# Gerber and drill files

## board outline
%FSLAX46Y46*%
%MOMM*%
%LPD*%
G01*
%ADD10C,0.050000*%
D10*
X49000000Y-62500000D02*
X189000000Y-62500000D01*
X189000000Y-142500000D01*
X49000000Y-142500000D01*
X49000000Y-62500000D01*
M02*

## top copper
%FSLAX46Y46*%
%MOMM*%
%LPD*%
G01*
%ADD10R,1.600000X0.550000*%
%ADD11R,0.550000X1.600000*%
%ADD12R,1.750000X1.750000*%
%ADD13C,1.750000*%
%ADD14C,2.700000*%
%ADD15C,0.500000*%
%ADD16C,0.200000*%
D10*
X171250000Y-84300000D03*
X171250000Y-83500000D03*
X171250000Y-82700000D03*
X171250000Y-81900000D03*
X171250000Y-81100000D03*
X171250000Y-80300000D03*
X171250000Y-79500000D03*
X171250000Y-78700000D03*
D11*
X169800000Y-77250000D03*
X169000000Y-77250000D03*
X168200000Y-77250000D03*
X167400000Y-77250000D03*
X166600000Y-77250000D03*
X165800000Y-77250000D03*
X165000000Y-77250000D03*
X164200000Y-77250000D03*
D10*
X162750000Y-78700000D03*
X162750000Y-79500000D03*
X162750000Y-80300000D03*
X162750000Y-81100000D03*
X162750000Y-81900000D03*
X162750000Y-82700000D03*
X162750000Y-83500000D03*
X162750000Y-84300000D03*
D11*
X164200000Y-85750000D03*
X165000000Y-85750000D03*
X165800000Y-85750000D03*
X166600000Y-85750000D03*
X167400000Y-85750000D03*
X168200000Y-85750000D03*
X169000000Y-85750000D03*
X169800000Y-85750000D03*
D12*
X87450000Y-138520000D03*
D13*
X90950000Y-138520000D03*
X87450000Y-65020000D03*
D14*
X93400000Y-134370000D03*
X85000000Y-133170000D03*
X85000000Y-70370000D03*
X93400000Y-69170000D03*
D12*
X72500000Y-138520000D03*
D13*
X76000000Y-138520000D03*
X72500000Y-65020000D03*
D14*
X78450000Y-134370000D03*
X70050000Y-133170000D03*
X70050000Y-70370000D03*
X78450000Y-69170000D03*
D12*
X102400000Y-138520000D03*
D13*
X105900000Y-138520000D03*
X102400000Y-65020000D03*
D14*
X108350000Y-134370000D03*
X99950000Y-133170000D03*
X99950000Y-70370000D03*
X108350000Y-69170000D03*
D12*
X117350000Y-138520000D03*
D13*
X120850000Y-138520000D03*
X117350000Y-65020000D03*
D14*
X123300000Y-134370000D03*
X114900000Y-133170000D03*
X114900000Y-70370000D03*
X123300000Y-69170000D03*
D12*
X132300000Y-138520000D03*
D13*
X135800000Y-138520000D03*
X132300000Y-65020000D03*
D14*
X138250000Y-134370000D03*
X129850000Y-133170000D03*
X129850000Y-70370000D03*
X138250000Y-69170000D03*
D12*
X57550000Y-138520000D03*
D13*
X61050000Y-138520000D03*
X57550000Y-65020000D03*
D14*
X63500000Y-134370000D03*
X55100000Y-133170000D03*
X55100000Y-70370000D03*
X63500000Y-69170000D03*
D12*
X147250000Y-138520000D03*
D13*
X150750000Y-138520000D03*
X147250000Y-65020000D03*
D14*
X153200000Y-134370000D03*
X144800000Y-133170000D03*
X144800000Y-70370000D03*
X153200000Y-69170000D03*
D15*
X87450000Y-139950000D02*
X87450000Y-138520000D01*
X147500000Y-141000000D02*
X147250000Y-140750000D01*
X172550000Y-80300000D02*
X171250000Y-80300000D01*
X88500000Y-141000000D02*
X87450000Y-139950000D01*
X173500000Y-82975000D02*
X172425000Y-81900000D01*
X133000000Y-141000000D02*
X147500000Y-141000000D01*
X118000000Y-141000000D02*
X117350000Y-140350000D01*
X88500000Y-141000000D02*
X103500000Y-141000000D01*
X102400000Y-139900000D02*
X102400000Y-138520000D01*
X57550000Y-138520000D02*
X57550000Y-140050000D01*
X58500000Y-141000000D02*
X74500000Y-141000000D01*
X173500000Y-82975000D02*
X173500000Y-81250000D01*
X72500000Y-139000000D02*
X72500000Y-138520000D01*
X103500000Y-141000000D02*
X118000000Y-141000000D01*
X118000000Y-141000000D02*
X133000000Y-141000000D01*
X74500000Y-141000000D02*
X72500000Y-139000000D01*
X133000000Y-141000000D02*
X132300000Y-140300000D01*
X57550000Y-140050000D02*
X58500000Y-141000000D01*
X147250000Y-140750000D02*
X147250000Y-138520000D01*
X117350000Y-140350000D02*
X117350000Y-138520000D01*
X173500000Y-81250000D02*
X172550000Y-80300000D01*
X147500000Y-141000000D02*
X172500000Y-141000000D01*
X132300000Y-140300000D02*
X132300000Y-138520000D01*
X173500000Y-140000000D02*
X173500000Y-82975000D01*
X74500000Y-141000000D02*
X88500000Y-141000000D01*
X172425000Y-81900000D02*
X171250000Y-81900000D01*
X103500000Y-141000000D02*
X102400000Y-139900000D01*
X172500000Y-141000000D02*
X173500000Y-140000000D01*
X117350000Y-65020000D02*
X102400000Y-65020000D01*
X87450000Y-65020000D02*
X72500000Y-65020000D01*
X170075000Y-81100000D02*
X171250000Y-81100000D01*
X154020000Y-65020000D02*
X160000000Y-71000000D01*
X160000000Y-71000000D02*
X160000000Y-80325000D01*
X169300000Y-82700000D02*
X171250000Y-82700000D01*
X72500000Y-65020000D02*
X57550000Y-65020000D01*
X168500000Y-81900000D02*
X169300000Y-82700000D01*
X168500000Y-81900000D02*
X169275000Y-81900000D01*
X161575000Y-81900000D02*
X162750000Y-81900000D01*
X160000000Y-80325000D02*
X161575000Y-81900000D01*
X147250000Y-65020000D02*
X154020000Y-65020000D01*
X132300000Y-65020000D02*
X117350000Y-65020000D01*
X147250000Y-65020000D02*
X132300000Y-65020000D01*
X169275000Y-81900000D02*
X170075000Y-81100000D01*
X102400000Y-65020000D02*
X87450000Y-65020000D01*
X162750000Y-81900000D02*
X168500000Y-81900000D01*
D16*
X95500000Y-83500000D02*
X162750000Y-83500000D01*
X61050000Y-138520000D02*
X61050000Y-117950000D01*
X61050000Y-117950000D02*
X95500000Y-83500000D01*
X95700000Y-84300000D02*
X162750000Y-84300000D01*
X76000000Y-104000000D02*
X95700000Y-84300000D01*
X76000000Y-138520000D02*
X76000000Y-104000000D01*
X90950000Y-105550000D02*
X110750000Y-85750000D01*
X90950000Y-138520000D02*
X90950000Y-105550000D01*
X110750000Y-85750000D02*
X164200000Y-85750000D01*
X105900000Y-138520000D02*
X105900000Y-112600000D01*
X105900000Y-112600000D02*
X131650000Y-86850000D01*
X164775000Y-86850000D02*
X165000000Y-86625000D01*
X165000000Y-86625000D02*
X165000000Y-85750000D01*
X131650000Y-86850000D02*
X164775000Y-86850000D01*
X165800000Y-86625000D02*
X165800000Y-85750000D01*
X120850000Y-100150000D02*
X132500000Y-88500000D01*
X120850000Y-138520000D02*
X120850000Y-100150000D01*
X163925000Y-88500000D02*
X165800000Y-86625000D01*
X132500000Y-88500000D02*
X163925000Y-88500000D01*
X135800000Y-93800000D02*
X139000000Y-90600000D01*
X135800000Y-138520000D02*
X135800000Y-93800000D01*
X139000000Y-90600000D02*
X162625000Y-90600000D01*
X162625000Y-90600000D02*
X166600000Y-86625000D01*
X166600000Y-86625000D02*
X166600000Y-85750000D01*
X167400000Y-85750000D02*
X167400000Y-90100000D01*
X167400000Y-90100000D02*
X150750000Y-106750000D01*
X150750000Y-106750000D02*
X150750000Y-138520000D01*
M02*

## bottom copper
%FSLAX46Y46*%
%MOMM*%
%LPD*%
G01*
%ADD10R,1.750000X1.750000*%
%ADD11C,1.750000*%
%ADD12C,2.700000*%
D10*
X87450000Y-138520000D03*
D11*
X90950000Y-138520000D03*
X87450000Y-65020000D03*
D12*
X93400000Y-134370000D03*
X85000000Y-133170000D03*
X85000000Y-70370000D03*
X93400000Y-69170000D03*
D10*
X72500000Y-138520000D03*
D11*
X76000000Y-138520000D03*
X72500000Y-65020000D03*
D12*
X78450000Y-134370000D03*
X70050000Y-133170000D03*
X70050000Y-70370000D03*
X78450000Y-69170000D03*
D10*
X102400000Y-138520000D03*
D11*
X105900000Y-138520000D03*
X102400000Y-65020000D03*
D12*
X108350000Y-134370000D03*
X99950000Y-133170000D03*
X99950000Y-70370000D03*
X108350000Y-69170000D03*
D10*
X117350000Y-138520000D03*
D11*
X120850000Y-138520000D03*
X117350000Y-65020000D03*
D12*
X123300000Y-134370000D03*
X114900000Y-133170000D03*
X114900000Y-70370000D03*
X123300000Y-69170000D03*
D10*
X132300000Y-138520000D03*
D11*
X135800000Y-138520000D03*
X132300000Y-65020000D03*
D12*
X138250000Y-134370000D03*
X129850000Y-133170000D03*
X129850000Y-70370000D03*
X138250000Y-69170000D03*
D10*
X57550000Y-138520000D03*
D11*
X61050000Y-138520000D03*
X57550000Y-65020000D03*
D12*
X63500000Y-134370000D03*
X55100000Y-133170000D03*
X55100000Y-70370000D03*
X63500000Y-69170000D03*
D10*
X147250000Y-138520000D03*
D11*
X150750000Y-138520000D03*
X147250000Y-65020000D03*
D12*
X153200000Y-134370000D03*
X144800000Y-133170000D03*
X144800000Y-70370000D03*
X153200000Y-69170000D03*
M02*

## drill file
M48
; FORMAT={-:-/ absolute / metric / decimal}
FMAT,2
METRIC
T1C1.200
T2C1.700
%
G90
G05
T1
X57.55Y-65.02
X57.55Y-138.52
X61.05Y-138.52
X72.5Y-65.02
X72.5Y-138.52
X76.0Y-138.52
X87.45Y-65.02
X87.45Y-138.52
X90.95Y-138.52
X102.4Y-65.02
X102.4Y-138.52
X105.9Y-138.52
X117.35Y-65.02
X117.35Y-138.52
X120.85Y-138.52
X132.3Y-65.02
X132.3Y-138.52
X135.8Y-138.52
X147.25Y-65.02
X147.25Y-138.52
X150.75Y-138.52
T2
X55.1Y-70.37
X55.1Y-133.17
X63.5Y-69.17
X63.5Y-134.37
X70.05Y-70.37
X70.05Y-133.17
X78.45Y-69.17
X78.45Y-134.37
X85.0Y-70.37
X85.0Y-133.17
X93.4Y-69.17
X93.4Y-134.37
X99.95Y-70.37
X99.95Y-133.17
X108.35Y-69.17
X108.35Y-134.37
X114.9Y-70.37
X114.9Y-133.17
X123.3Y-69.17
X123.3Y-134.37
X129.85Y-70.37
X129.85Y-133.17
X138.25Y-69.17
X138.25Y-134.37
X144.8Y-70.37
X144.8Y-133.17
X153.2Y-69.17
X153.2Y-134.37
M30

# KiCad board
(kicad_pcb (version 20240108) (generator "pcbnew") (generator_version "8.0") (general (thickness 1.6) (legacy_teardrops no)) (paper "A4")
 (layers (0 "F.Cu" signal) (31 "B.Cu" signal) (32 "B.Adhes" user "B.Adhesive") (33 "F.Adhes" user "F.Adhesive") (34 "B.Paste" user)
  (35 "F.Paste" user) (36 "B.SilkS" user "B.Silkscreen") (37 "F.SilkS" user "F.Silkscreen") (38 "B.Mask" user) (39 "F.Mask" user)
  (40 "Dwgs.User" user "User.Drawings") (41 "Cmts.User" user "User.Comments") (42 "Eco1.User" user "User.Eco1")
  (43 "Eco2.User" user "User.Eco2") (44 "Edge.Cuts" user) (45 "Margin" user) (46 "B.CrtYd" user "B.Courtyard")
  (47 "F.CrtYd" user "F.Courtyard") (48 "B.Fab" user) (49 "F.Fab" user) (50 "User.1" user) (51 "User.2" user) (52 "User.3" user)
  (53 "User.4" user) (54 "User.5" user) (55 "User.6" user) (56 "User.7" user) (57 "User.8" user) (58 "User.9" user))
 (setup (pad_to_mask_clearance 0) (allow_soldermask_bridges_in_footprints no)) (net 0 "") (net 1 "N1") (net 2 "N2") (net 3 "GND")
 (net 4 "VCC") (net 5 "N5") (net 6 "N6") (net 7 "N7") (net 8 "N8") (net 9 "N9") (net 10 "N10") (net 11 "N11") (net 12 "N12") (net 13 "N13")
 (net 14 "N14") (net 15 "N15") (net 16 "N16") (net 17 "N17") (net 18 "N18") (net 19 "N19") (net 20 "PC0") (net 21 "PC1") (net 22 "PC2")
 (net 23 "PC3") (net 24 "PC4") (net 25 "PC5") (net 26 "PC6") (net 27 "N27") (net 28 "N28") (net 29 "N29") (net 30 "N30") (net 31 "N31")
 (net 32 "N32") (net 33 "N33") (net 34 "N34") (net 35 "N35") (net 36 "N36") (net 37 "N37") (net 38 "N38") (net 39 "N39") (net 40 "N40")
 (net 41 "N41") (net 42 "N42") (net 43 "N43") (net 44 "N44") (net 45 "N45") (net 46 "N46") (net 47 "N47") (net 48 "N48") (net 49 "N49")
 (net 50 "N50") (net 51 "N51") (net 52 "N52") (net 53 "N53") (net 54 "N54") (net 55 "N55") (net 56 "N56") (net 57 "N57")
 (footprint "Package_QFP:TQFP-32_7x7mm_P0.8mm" (layer "F.Cu") (at 167 81.5 180)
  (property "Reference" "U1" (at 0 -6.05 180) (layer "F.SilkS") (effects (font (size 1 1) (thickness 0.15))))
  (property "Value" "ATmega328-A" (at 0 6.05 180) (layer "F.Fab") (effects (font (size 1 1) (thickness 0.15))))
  (pad "1" smd rect (at -4.25 -2.8 180) (size 1.6 0.55) (layers "F.Cu" "F.Paste" "F.Mask") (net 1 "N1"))
  (pad "2" smd rect (at -4.25 -2 180) (size 1.6 0.55) (layers "F.Cu" "F.Paste" "F.Mask") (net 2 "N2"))
  (pad "3" smd rect (at -4.25 -1.2 180) (size 1.6 0.55) (layers "F.Cu" "F.Paste" "F.Mask") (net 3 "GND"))
  (pad "4" smd rect (at -4.25 -0.4 180) (size 1.6 0.55) (layers "F.Cu" "F.Paste" "F.Mask") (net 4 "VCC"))
  (pad "5" smd rect (at -4.25 0.4 180) (size 1.6 0.55) (layers "F.Cu" "F.Paste" "F.Mask") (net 3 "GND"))
  (pad "6" smd rect (at -4.25 1.2 180) (size 1.6 0.55) (layers "F.Cu" "F.Paste" "F.Mask") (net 4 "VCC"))
  (pad "7" smd rect (at -4.25 2 180) (size 1.6 0.55) (layers "F.Cu" "F.Paste" "F.Mask") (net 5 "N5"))
  (pad "8" smd rect (at -4.25 2.8 180) (size 1.6 0.55) (layers "F.Cu" "F.Paste" "F.Mask") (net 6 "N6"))
  (pad "9" smd rect (at -2.8 4.25 270) (size 1.6 0.55) (layers "F.Cu" "F.Paste" "F.Mask") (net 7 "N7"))
  (pad "10" smd rect (at -2 4.25 270) (size 1.6 0.55) (layers "F.Cu" "F.Paste" "F.Mask") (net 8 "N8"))
  (pad "11" smd rect (at -1.2 4.25 270) (size 1.6 0.55) (layers "F.Cu" "F.Paste" "F.Mask") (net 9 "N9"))
  (pad "12" smd rect (at -0.4 4.25 270) (size 1.6 0.55) (layers "F.Cu" "F.Paste" "F.Mask") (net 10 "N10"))
  (pad "13" smd rect (at 0.4 4.25 270) (size 1.6 0.55) (layers "F.Cu" "F.Paste" "F.Mask") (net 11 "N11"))
  (pad "14" smd rect (at 1.2 4.25 270) (size 1.6 0.55) (layers "F.Cu" "F.Paste" "F.Mask") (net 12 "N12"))
  (pad "15" smd rect (at 2 4.25 270) (size 1.6 0.55) (layers "F.Cu" "F.Paste" "F.Mask") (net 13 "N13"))
  (pad "16" smd rect (at 2.8 4.25 270) (size 1.6 0.55) (layers "F.Cu" "F.Paste" "F.Mask") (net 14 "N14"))
  (pad "17" smd rect (at 4.25 2.8 180) (size 1.6 0.55) (layers "F.Cu" "F.Paste" "F.Mask") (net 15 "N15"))
  (pad "18" smd rect (at 4.25 2 180) (size 1.6 0.55) (layers "F.Cu" "F.Paste" "F.Mask") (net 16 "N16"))
  (pad "19" smd rect (at 4.25 1.2 180) (size 1.6 0.55) (layers "F.Cu" "F.Paste" "F.Mask") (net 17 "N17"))
  (pad "20" smd rect (at 4.25 0.4 180) (size 1.6 0.55) (layers "F.Cu" "F.Paste" "F.Mask") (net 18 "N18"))
  (pad "21" smd rect (at 4.25 -0.4 180) (size 1.6 0.55) (layers "F.Cu" "F.Paste" "F.Mask") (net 3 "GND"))
  (pad "22" smd rect (at 4.25 -1.2 180) (size 1.6 0.55) (layers "F.Cu" "F.Paste" "F.Mask") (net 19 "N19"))
  (pad "23" smd rect (at 4.25 -2 180) (size 1.6 0.55) (layers "F.Cu" "F.Paste" "F.Mask") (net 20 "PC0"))
  (pad "24" smd rect (at 4.25 -2.8 180) (size 1.6 0.55) (layers "F.Cu" "F.Paste" "F.Mask") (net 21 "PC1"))
  (pad "25" smd rect (at 2.8 -4.25 270) (size 1.6 0.55) (layers "F.Cu" "F.Paste" "F.Mask") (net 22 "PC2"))
  (pad "26" smd rect (at 2 -4.25 270) (size 1.6 0.55) (layers "F.Cu" "F.Paste" "F.Mask") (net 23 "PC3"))
  (pad "27" smd rect (at 1.2 -4.25 270) (size 1.6 0.55) (layers "F.Cu" "F.Paste" "F.Mask") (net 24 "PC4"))
  (pad "28" smd rect (at 0.4 -4.25 270) (size 1.6 0.55) (layers "F.Cu" "F.Paste" "F.Mask") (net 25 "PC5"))
  (pad "29" smd rect (at -0.4 -4.25 270) (size 1.6 0.55) (layers "F.Cu" "F.Paste" "F.Mask") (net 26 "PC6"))
  (pad "30" smd rect (at -1.2 -4.25 270) (size 1.6 0.55) (layers "F.Cu" "F.Paste" "F.Mask") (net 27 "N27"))
  (pad "31" smd rect (at -2 -4.25 270) (size 1.6 0.55) (layers "F.Cu" "F.Paste" "F.Mask") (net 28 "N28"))
  (pad "32" smd rect (at -2.8 -4.25 270) (size 1.6 0.55) (layers "F.Cu" "F.Paste" "F.Mask") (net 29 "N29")))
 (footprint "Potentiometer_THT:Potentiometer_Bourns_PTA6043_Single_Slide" (layer "F.Cu") (at 87.45 138.52 90)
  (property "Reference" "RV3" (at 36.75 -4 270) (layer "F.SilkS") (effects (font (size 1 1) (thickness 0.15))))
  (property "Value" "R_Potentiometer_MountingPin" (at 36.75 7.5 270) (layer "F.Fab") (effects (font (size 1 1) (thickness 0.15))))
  (pad "1" thru_hole rect (at 0 0 90) (size 1.75 1.75) (drill 1.2) (layers "*.Cu" "*.Mask") (remove_unused_layers no) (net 4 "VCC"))
  (pad "2" thru_hole circle (at 0 3.5 90) (size 1.75 1.75) (drill 1.2) (layers "*.Cu" "*.Mask") (remove_unused_layers no) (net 22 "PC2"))
  (pad "3" thru_hole circle (at 73.5 0 90) (size 1.75 1.75) (drill 1.2) (layers "*.Cu" "*.Mask") (remove_unused_layers no) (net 3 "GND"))
  (pad "MP" thru_hole circle (at 4.15 5.95 90) (size 2.7 2.7) (drill 1.7) (layers "*.Cu" "*.Mask") (remove_unused_layers no) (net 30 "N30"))
  (pad "MP" thru_hole circle (at 5.35 -2.45 90) (size 2.7 2.7) (drill 1.7) (layers "*.Cu" "*.Mask") (remove_unused_layers no) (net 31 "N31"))
  (pad "MP" thru_hole circle (at 68.15 -2.45 90) (size 2.7 2.7) (drill 1.7) (layers "*.Cu" "*.Mask") (remove_unused_layers no)
   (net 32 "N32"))
  (pad "MP" thru_hole circle (at 69.35 5.95 90) (size 2.7 2.7) (drill 1.7) (layers "*.Cu" "*.Mask") (remove_unused_layers no) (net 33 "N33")))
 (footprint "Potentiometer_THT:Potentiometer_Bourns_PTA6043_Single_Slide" (layer "F.Cu") (at 72.5 138.52 90)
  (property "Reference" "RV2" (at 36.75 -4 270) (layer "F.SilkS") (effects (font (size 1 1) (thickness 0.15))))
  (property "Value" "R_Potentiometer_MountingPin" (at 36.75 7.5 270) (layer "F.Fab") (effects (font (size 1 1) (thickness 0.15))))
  (pad "1" thru_hole rect (at 0 0 90) (size 1.75 1.75) (drill 1.2) (layers "*.Cu" "*.Mask") (remove_unused_layers no) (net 4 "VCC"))
  (pad "2" thru_hole circle (at 0 3.5 90) (size 1.75 1.75) (drill 1.2) (layers "*.Cu" "*.Mask") (remove_unused_layers no) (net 21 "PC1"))
  (pad "3" thru_hole circle (at 73.5 0 90) (size 1.75 1.75) (drill 1.2) (layers "*.Cu" "*.Mask") (remove_unused_layers no) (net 3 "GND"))
  (pad "MP" thru_hole circle (at 4.15 5.95 90) (size 2.7 2.7) (drill 1.7) (layers "*.Cu" "*.Mask") (remove_unused_layers no) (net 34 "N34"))
  (pad "MP" thru_hole circle (at 5.35 -2.45 90) (size 2.7 2.7) (drill 1.7) (layers "*.Cu" "*.Mask") (remove_unused_layers no) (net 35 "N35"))
  (pad "MP" thru_hole circle (at 68.15 -2.45 90) (size 2.7 2.7) (drill 1.7) (layers "*.Cu" "*.Mask") (remove_unused_layers no)
   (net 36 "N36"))
  (pad "MP" thru_hole circle (at 69.35 5.95 90) (size 2.7 2.7) (drill 1.7) (layers "*.Cu" "*.Mask") (remove_unused_layers no) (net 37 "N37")))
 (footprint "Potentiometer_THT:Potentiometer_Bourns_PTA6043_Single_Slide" (layer "F.Cu") (at 102.4 138.52 90)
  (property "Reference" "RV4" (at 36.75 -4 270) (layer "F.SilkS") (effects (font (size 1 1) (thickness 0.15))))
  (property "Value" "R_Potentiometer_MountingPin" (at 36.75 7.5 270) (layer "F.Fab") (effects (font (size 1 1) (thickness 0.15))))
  (pad "1" thru_hole rect (at 0 0 90) (size 1.75 1.75) (drill 1.2) (layers "*.Cu" "*.Mask") (remove_unused_layers no) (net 4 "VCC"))
  (pad "2" thru_hole circle (at 0 3.5 90) (size 1.75 1.75) (drill 1.2) (layers "*.Cu" "*.Mask") (remove_unused_layers no) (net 23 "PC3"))
  (pad "3" thru_hole circle (at 73.5 0 90) (size 1.75 1.75) (drill 1.2) (layers "*.Cu" "*.Mask") (remove_unused_layers no) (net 3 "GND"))
  (pad "MP" thru_hole circle (at 4.15 5.95 90) (size 2.7 2.7) (drill 1.7) (layers "*.Cu" "*.Mask") (remove_unused_layers no) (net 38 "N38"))
  (pad "MP" thru_hole circle (at 5.35 -2.45 90) (size 2.7 2.7) (drill 1.7) (layers "*.Cu" "*.Mask") (remove_unused_layers no) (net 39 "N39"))
  (pad "MP" thru_hole circle (at 68.15 -2.45 90) (size 2.7 2.7) (drill 1.7) (layers "*.Cu" "*.Mask") (remove_unused_layers no)
   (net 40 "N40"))
  (pad "MP" thru_hole circle (at 69.35 5.95 90) (size 2.7 2.7) (drill 1.7) (layers "*.Cu" "*.Mask") (remove_unused_layers no) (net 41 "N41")))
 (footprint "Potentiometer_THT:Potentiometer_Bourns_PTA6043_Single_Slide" (layer "F.Cu") (at 117.35 138.52 90)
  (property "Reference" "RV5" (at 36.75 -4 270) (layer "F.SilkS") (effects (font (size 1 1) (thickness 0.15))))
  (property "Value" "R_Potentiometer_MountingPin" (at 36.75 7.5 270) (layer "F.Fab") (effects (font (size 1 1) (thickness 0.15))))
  (pad "1" thru_hole rect (at 0 0 90) (size 1.75 1.75) (drill 1.2) (layers "*.Cu" "*.Mask") (remove_unused_layers no) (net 4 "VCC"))
  (pad "2" thru_hole circle (at 0 3.5 90) (size 1.75 1.75) (drill 1.2) (layers "*.Cu" "*.Mask") (remove_unused_layers no) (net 24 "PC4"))
  (pad "3" thru_hole circle (at 73.5 0 90) (size 1.75 1.75) (drill 1.2) (layers "*.Cu" "*.Mask") (remove_unused_layers no) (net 3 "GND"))
  (pad "MP" thru_hole circle (at 4.15 5.95 90) (size 2.7 2.7) (drill 1.7) (layers "*.Cu" "*.Mask") (remove_unused_layers no) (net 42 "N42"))
  (pad "MP" thru_hole circle (at 5.35 -2.45 90) (size 2.7 2.7) (drill 1.7) (layers "*.Cu" "*.Mask") (remove_unused_layers no) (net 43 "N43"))
  (pad "MP" thru_hole circle (at 68.15 -2.45 90) (size 2.7 2.7) (drill 1.7) (layers "*.Cu" "*.Mask") (remove_unused_layers no)
   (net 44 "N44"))
  (pad "MP" thru_hole circle (at 69.35 5.95 90) (size 2.7 2.7) (drill 1.7) (layers "*.Cu" "*.Mask") (remove_unused_layers no) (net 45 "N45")))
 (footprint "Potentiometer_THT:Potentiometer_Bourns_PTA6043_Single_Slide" (layer "F.Cu") (at 132.3 138.52 90)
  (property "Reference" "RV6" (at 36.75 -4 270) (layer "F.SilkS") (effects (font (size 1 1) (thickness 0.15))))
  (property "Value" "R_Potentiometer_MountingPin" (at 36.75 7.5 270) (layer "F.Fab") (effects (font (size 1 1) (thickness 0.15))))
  (pad "1" thru_hole rect (at 0 0 90) (size 1.75 1.75) (drill 1.2) (layers "*.Cu" "*.Mask") (remove_unused_layers no) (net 4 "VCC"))
  (pad "2" thru_hole circle (at 0 3.5 90) (size 1.75 1.75) (drill 1.2) (layers "*.Cu" "*.Mask") (remove_unused_layers no) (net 25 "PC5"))
  (pad "3" thru_hole circle (at 73.5 0 90) (size 1.75 1.75) (drill 1.2) (layers "*.Cu" "*.Mask") (remove_unused_layers no) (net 3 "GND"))
  (pad "MP" thru_hole circle (at 4.15 5.95 90) (size 2.7 2.7) (drill 1.7) (layers "*.Cu" "*.Mask") (remove_unused_layers no) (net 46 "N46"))
  (pad "MP" thru_hole circle (at 5.35 -2.45 90) (size 2.7 2.7) (drill 1.7) (layers "*.Cu" "*.Mask") (remove_unused_layers no) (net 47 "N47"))
  (pad "MP" thru_hole circle (at 68.15 -2.45 90) (size 2.7 2.7) (drill 1.7) (layers "*.Cu" "*.Mask") (remove_unused_layers no)
   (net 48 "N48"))
  (pad "MP" thru_hole circle (at 69.35 5.95 90) (size 2.7 2.7) (drill 1.7) (layers "*.Cu" "*.Mask") (remove_unused_layers no) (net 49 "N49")))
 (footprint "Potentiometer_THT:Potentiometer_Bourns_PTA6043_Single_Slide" (layer "F.Cu") (at 57.55 138.52 90)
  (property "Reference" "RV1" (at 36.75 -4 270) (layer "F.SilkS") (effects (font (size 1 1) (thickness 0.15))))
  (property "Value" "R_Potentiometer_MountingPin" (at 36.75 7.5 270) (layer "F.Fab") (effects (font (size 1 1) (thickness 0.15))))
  (pad "1" thru_hole rect (at 0 0 90) (size 1.75 1.75) (drill 1.2) (layers "*.Cu" "*.Mask") (remove_unused_layers no) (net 4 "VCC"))
  (pad "2" thru_hole circle (at 0 3.5 90) (size 1.75 1.75) (drill 1.2) (layers "*.Cu" "*.Mask") (remove_unused_layers no) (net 20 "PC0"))
  (pad "3" thru_hole circle (at 73.5 0 90) (size 1.75 1.75) (drill 1.2) (layers "*.Cu" "*.Mask") (remove_unused_layers no) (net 3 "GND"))
  (pad "MP" thru_hole circle (at 4.15 5.95 90) (size 2.7 2.7) (drill 1.7) (layers "*.Cu" "*.Mask") (remove_unused_layers no) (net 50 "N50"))
  (pad "MP" thru_hole circle (at 5.35 -2.45 90) (size 2.7 2.7) (drill 1.7) (layers "*.Cu" "*.Mask") (remove_unused_layers no) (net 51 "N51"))
  (pad "MP" thru_hole circle (at 68.15 -2.45 90) (size 2.7 2.7) (drill 1.7) (layers "*.Cu" "*.Mask") (remove_unused_layers no)
   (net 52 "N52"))
  (pad "MP" thru_hole circle (at 69.35 5.95 90) (size 2.7 2.7) (drill 1.7) (layers "*.Cu" "*.Mask") (remove_unused_layers no) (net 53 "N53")))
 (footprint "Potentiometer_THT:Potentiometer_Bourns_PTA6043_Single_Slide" (layer "F.Cu") (at 147.25 138.52 90)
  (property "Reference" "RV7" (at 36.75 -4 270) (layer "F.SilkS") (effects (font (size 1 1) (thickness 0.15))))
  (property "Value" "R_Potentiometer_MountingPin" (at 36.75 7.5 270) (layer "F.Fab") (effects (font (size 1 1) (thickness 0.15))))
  (pad "1" thru_hole rect (at 0 0 90) (size 1.75 1.75) (drill 1.2) (layers "*.Cu" "*.Mask") (remove_unused_layers no) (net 4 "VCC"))
  (pad "2" thru_hole circle (at 0 3.5 90) (size 1.75 1.75) (drill 1.2) (layers "*.Cu" "*.Mask") (remove_unused_layers no) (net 26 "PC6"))
  (pad "3" thru_hole circle (at 73.5 0 90) (size 1.75 1.75) (drill 1.2) (layers "*.Cu" "*.Mask") (remove_unused_layers no) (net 3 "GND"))
  (pad "MP" thru_hole circle (at 4.15 5.95 90) (size 2.7 2.7) (drill 1.7) (layers "*.Cu" "*.Mask") (remove_unused_layers no) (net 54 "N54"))
  (pad "MP" thru_hole circle (at 5.35 -2.45 90) (size 2.7 2.7) (drill 1.7) (layers "*.Cu" "*.Mask") (remove_unused_layers no) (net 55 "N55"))
  (pad "MP" thru_hole circle (at 68.15 -2.45 90) (size 2.7 2.7) (drill 1.7) (layers "*.Cu" "*.Mask") (remove_unused_layers no)
   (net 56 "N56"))
  (pad "MP" thru_hole circle (at 69.35 5.95 90) (size 2.7 2.7) (drill 1.7) (layers "*.Cu" "*.Mask") (remove_unused_layers no) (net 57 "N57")))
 (gr_rect (start 49 62.5) (end 189 142.5) (stroke (width 0.05) (type default)) (fill none) (layer "Edge.Cuts"))
 (segment (start 87.45 139.95) (end 87.45 138.52) (width 0.5) (layer "F.Cu") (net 4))
 (segment (start 147.5 141) (end 147.25 140.75) (width 0.5) (layer "F.Cu") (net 4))
 (segment (start 172.55 80.3) (end 171.25 80.3) (width 0.5) (layer "F.Cu") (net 4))
 (segment (start 88.5 141) (end 87.45 139.95) (width 0.5) (layer "F.Cu") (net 4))
 (segment (start 173.5 82.975) (end 172.425 81.9) (width 0.5) (layer "F.Cu") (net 4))
 (segment (start 133 141) (end 147.5 141) (width 0.5) (layer "F.Cu") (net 4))
 (segment (start 118 141) (end 117.35 140.35) (width 0.5) (layer "F.Cu") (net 4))
 (segment (start 88.5 141) (end 103.5 141) (width 0.5) (layer "F.Cu") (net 4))
 (segment (start 102.4 139.9) (end 102.4 138.52) (width 0.5) (layer "F.Cu") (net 4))
 (segment (start 57.55 138.52) (end 57.55 140.05) (width 0.5) (layer "F.Cu") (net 4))
 (segment (start 58.5 141) (end 74.5 141) (width 0.5) (layer "F.Cu") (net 4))
 (segment (start 173.5 82.975) (end 173.5 81.25) (width 0.5) (layer "F.Cu") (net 4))
 (segment (start 72.5 139) (end 72.5 138.52) (width 0.5) (layer "F.Cu") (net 4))
 (segment (start 103.5 141) (end 118 141) (width 0.5) (layer "F.Cu") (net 4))
 (segment (start 118 141) (end 133 141) (width 0.5) (layer "F.Cu") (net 4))
 (segment (start 74.5 141) (end 72.5 139) (width 0.5) (layer "F.Cu") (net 4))
 (segment (start 133 141) (end 132.3 140.3) (width 0.5) (layer "F.Cu") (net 4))
 (segment (start 57.55 140.05) (end 58.5 141) (width 0.5) (layer "F.Cu") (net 4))
 (segment (start 147.25 140.75) (end 147.25 138.52) (width 0.5) (layer "F.Cu") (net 4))
 (segment (start 117.35 140.35) (end 117.35 138.52) (width 0.5) (layer "F.Cu") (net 4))
 (segment (start 173.5 81.25) (end 172.55 80.3) (width 0.5) (layer "F.Cu") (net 4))
 (segment (start 147.5 141) (end 172.5 141) (width 0.5) (layer "F.Cu") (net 4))
 (segment (start 132.3 140.3) (end 132.3 138.52) (width 0.5) (layer "F.Cu") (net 4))
 (segment (start 173.5 140) (end 173.5 82.975) (width 0.5) (layer "F.Cu") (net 4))
 (segment (start 74.5 141) (end 88.5 141) (width 0.5) (layer "F.Cu") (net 4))
 (segment (start 172.425 81.9) (end 171.25 81.9) (width 0.5) (layer "F.Cu") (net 4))
 (segment (start 103.5 141) (end 102.4 139.9) (width 0.5) (layer "F.Cu") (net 4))
 (segment (start 172.5 141) (end 173.5 140) (width 0.5) (layer "F.Cu") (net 4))
 (segment (start 117.35 65.02) (end 102.4 65.02) (width 0.5) (layer "F.Cu") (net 3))
 (segment (start 87.45 65.02) (end 72.5 65.02) (width 0.5) (layer "F.Cu") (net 3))
 (segment (start 170.075 81.1) (end 171.25 81.1) (width 0.5) (layer "F.Cu") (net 3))
 (segment (start 154.02 65.02) (end 160 71) (width 0.5) (layer "F.Cu") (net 3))
 (segment (start 160 71) (end 160 80.325) (width 0.5) (layer "F.Cu") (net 3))
 (segment (start 169.3 82.7) (end 171.25 82.7) (width 0.5) (layer "F.Cu") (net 3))
 (segment (start 72.5 65.02) (end 57.55 65.02) (width 0.5) (layer "F.Cu") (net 3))
 (segment (start 168.5 81.9) (end 169.3 82.7) (width 0.5) (layer "F.Cu") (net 3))
 (segment (start 168.5 81.9) (end 169.275 81.9) (width 0.5) (layer "F.Cu") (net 3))
 (segment (start 161.575 81.9) (end 162.75 81.9) (width 0.5) (layer "F.Cu") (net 3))
 (segment (start 160 80.325) (end 161.575 81.9) (width 0.5) (layer "F.Cu") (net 3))
 (segment (start 147.25 65.02) (end 154.02 65.02) (width 0.5) (layer "F.Cu") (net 3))
 (segment (start 132.3 65.02) (end 117.35 65.02) (width 0.5) (layer "F.Cu") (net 3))
 (segment (start 147.25 65.02) (end 132.3 65.02) (width 0.5) (layer "F.Cu") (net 3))
 (segment (start 169.275 81.9) (end 170.075 81.1) (width 0.5) (layer "F.Cu") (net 3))
 (segment (start 102.4 65.02) (end 87.45 65.02) (width 0.5) (layer "F.Cu") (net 3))
 (segment (start 162.75 81.9) (end 168.5 81.9) (width 0.5) (layer "F.Cu") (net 3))
 (segment (start 95.5 83.5) (end 162.75 83.5) (width 0.2) (layer "F.Cu") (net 20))
 (segment (start 61.05 138.52) (end 61.05 117.95) (width 0.2) (layer "F.Cu") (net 20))
 (segment (start 61.05 117.95) (end 95.5 83.5) (width 0.2) (layer "F.Cu") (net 20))
 (segment (start 95.7 84.3) (end 162.75 84.3) (width 0.2) (layer "F.Cu") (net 21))
 (segment (start 76 104) (end 95.7 84.3) (width 0.2) (layer "F.Cu") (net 21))
 (segment (start 76 138.52) (end 76 104) (width 0.2) (layer "F.Cu") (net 21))
 (segment (start 90.95 105.55) (end 110.75 85.75) (width 0.2) (layer "F.Cu") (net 22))
 (segment (start 90.95 138.52) (end 90.95 105.55) (width 0.2) (layer "F.Cu") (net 22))
 (segment (start 110.75 85.75) (end 164.2 85.75) (width 0.2) (layer "F.Cu") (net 22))
 (segment (start 105.9 138.52) (end 105.9 112.6) (width 0.2) (layer "F.Cu") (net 23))
 (segment (start 105.9 112.6) (end 131.65 86.85) (width 0.2) (layer "F.Cu") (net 23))
 (segment (start 164.775 86.85) (end 165 86.625) (width 0.2) (layer "F.Cu") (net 23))
 (segment (start 165 86.625) (end 165 85.75) (width 0.2) (layer "F.Cu") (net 23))
 (segment (start 131.65 86.85) (end 164.775 86.85) (width 0.2) (layer "F.Cu") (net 23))
 (segment (start 165.8 86.625) (end 165.8 85.75) (width 0.2) (layer "F.Cu") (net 24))
 (segment (start 120.85 100.15) (end 132.5 88.5) (width 0.2) (layer "F.Cu") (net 24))
 (segment (start 120.85 138.52) (end 120.85 100.15) (width 0.2) (layer "F.Cu") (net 24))
 (segment (start 163.925 88.5) (end 165.8 86.625) (width 0.2) (layer "F.Cu") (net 24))
 (segment (start 132.5 88.5) (end 163.925 88.5) (width 0.2) (layer "F.Cu") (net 24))
 (segment (start 135.8 93.8) (end 139 90.6) (width 0.2) (layer "F.Cu") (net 25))
 (segment (start 135.8 138.52) (end 135.8 93.8) (width 0.2) (layer "F.Cu") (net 25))
 (segment (start 139 90.6) (end 162.625 90.6) (width 0.2) (layer "F.Cu") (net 25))
 (segment (start 162.625 90.6) (end 166.6 86.625) (width 0.2) (layer "F.Cu") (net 25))
 (segment (start 166.6 86.625) (end 166.6 85.75) (width 0.2) (layer "F.Cu") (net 25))
 (segment (start 167.4 85.75) (end 167.4 90.1) (width 0.2) (layer "F.Cu") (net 26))
 (segment (start 167.4 90.1) (end 150.75 106.75) (width 0.2) (layer "F.Cu") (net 26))
 (segment (start 150.75 106.75) (end 150.75 138.52) (width 0.2) (layer "F.Cu") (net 26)))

